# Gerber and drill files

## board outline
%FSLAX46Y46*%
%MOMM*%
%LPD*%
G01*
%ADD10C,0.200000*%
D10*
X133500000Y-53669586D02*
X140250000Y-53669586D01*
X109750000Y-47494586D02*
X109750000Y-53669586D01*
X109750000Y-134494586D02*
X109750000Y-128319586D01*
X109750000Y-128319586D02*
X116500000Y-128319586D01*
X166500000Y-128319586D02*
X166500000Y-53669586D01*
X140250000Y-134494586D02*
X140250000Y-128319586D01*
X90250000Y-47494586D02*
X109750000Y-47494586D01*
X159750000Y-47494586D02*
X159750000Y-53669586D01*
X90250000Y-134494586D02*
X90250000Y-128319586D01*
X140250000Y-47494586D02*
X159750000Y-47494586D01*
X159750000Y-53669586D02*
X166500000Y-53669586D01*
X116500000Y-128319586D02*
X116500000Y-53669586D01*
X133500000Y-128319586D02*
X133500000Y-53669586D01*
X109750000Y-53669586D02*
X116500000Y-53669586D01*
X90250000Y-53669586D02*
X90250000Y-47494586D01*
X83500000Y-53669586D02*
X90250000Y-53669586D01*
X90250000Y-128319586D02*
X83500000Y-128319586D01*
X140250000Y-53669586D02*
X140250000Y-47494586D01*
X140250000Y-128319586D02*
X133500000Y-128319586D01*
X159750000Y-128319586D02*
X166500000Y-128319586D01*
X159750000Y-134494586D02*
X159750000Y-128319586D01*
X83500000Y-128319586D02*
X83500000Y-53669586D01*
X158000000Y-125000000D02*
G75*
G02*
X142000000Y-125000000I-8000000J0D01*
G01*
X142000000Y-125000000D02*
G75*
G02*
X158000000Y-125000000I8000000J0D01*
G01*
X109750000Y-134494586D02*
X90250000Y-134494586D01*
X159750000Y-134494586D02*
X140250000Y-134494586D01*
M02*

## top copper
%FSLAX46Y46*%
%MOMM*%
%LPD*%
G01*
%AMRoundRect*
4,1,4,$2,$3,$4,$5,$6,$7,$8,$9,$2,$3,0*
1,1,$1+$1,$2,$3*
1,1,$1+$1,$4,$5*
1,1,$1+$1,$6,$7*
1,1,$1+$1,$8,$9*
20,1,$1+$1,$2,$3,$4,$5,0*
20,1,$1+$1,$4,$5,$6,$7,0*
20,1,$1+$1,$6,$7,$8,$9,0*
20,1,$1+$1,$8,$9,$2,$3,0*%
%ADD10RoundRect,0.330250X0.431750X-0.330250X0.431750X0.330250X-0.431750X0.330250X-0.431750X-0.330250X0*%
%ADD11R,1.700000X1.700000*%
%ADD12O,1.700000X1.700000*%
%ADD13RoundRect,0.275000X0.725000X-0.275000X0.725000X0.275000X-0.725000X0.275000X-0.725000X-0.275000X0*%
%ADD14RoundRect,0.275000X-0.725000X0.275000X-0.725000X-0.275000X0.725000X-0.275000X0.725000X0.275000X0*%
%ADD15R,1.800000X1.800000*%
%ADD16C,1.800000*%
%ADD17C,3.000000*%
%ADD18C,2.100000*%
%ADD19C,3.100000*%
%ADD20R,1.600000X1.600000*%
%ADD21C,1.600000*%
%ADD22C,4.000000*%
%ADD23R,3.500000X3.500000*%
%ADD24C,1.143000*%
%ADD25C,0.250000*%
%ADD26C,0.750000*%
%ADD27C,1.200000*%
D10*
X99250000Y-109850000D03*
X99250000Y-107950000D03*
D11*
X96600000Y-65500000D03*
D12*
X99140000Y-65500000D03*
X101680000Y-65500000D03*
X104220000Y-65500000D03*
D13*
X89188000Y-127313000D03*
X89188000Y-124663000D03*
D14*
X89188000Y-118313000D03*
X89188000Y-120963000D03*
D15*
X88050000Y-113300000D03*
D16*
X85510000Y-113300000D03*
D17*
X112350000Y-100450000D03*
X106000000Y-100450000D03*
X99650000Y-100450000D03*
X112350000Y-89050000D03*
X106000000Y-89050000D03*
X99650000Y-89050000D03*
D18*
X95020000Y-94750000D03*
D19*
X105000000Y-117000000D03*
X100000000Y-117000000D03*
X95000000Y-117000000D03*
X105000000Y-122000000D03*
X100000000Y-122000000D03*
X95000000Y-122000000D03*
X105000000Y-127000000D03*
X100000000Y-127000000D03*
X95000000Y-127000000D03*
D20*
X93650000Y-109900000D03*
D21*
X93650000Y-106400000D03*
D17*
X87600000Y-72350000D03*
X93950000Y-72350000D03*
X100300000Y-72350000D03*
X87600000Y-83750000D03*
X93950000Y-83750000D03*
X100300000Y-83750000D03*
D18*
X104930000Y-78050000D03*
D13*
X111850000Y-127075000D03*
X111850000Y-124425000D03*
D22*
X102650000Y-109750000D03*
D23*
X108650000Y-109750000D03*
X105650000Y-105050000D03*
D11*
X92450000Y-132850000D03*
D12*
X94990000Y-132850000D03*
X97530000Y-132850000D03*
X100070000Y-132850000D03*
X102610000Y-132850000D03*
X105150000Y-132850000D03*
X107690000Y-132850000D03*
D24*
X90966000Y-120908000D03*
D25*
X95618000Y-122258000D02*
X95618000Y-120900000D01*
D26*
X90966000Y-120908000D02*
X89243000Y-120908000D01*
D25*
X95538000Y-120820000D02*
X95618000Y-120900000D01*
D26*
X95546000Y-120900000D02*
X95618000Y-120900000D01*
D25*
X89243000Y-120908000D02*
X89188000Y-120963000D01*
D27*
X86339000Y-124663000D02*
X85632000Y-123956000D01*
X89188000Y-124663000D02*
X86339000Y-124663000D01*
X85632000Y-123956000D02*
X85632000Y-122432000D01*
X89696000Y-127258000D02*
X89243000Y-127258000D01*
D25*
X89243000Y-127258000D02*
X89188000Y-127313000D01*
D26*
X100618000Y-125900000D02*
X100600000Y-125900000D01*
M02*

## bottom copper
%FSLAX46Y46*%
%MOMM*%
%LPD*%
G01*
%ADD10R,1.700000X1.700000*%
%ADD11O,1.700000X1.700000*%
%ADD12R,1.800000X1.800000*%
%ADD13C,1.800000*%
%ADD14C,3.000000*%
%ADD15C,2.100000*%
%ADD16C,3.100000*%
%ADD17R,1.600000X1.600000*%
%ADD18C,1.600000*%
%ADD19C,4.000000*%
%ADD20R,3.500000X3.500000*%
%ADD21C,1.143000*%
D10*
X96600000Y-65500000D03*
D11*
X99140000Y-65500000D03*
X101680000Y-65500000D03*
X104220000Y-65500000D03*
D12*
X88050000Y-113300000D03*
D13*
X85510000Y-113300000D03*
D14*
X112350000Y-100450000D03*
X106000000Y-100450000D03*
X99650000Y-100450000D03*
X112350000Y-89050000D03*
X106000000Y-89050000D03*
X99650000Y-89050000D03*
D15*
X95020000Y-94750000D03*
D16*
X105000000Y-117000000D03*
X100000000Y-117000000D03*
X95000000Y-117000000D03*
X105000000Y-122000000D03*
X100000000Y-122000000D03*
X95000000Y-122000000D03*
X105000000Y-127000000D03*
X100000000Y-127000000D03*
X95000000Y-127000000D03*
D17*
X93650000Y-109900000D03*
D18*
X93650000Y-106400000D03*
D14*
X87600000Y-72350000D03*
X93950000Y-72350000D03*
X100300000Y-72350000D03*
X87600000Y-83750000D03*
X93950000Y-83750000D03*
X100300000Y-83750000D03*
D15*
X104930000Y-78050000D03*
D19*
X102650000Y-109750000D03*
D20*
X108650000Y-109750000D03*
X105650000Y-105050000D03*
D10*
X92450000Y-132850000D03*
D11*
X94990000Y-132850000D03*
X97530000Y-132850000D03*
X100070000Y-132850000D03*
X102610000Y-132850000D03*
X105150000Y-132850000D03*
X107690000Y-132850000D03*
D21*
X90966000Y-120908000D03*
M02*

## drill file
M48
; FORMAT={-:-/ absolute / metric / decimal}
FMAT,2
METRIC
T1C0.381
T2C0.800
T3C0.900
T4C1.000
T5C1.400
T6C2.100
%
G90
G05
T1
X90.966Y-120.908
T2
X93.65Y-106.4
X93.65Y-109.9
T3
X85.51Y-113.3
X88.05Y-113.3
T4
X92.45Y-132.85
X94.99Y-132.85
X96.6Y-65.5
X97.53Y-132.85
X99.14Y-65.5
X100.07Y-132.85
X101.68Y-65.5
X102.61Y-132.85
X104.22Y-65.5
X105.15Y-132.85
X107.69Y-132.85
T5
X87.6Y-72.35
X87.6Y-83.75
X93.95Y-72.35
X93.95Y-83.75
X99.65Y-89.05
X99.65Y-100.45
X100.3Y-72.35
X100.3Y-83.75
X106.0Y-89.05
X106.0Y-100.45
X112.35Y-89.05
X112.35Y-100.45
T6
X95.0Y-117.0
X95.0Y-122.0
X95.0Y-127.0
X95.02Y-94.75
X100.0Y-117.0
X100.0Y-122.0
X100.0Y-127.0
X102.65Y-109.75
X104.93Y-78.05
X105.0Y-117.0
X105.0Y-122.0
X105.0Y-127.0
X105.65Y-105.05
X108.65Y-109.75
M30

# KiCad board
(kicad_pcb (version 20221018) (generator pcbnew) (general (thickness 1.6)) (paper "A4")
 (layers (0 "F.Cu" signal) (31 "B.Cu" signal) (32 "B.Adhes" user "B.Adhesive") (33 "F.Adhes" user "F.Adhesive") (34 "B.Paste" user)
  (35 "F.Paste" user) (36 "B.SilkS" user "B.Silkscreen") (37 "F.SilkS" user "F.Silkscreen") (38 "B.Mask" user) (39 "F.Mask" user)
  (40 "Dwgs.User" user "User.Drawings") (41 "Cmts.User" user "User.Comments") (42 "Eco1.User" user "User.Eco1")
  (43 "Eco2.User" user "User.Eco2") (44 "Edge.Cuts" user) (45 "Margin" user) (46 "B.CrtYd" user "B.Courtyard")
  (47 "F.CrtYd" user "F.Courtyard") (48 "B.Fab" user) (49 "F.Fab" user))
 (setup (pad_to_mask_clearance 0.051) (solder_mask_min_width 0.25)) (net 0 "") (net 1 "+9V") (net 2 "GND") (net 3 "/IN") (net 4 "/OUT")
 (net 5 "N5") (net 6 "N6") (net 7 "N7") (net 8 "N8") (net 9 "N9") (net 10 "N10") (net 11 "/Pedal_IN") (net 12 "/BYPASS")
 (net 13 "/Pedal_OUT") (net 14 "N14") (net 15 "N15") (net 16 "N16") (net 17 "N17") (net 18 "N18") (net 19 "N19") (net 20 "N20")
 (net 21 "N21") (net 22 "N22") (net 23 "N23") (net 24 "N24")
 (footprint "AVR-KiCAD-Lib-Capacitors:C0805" (layer "F.Cu") (at 99.25 108.9 90)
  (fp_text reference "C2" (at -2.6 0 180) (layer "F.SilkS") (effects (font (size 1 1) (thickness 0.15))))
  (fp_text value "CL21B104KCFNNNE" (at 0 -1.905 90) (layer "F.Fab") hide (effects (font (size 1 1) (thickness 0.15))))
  (pad "1" smd roundrect (at -0.95 0 90) (size 1.321 1.524) (layers "F.Cu" "F.Paste" "F.Mask") (roundrect_rratio 0.25) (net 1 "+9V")
   (solder_mask_margin 0.102))
  (pad "2" smd roundrect (at 0.95 0 90) (size 1.321 1.524) (layers "F.Cu" "F.Paste" "F.Mask") (roundrect_rratio 0.25) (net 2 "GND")
   (solder_mask_margin 0.102)))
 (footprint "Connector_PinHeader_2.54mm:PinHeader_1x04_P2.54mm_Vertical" (layer "F.Cu") (at 96.6 65.5 90)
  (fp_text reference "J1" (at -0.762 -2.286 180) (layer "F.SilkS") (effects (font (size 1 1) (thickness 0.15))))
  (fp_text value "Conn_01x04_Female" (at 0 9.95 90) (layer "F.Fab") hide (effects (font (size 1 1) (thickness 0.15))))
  (pad "1" thru_hole rect (at 0 0 90) (size 1.7 1.7) (drill 1) (layers "*.Cu" "*.Mask") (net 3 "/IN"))
  (pad "2" thru_hole oval (at 0 2.54 90) (size 1.7 1.7) (drill 1) (layers "*.Cu" "*.Mask") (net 2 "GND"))
  (pad "3" thru_hole oval (at 0 5.08 90) (size 1.7 1.7) (drill 1) (layers "*.Cu" "*.Mask") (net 1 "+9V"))
  (pad "4" thru_hole oval (at 0 7.62 90) (size 1.7 1.7) (drill 1) (layers "*.Cu" "*.Mask") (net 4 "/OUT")))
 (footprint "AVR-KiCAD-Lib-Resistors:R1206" (layer "F.Cu") (at 89.188 125.988 90)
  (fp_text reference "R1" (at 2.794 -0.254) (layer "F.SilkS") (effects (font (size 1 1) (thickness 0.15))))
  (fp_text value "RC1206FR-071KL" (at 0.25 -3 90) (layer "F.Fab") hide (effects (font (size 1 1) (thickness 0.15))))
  (pad "1" smd roundrect (at -1.325 0 90) (size 1.1 2) (layers "F.Cu" "F.Paste" "F.Mask") (roundrect_rratio 0.25) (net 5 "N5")
   (solder_mask_margin 0.102))
  (pad "2" smd roundrect (at 1.325 0 90) (size 1.1 2) (layers "F.Cu" "F.Paste" "F.Mask") (roundrect_rratio 0.25) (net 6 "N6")
   (solder_mask_margin 0.102)))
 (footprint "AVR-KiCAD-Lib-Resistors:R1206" (layer "F.Cu") (at 89.188 119.638 -90)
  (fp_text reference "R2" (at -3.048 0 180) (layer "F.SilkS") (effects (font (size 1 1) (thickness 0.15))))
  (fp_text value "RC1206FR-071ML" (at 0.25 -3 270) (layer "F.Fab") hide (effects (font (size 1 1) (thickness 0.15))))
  (pad "1" smd roundrect (at -1.325 0 270) (size 1.1 2) (layers "F.Cu" "F.Paste" "F.Mask") (roundrect_rratio 0.25) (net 3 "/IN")
   (solder_mask_margin 0.102))
  (pad "2" smd roundrect (at 1.325 0 270) (size 1.1 2) (layers "F.Cu" "F.Paste" "F.Mask") (roundrect_rratio 0.25) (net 2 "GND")
   (solder_mask_margin 0.102)))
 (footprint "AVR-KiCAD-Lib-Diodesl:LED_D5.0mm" (layer "F.Cu") (at 88.05 113.3 180)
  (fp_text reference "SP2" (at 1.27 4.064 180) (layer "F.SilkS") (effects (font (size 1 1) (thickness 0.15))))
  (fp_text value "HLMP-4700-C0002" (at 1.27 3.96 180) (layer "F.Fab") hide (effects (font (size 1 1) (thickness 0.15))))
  (pad "1" thru_hole rect (at 0 0 180) (size 1.8 1.8) (drill 0.9) (layers "*.Cu" "*.Mask") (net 6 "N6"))
  (pad "2" thru_hole circle (at 2.54 0 180) (size 1.8 1.8) (drill 0.9) (layers "*.Cu" "*.Mask") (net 1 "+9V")))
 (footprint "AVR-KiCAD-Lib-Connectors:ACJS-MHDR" (layer "F.Cu") (at 106 94.75)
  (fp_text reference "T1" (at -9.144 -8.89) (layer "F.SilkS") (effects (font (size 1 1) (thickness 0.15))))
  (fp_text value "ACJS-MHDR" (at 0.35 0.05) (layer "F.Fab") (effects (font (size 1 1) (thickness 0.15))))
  (pad "1" thru_hole circle (at 6.35 5.7) (size 3 3) (drill 1.4) (layers "*.Cu" "*.Mask") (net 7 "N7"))
  (pad "2" thru_hole circle (at 0 5.7) (size 3 3) (drill 1.4) (layers "*.Cu" "*.Mask") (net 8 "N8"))
  (pad "3" thru_hole circle (at -6.35 5.7) (size 3 3) (drill 1.4) (layers "*.Cu" "*.Mask") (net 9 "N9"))
  (pad "4" thru_hole circle (at 6.35 -5.7) (size 3 3) (drill 1.4) (layers "*.Cu" "*.Mask") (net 2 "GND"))
  (pad "5" thru_hole circle (at 0 -5.7) (size 3 3) (drill 1.4) (layers "*.Cu" "*.Mask") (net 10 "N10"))
  (pad "6" thru_hole circle (at -6.35 -5.7) (size 3 3) (drill 1.4) (layers "*.Cu" "*.Mask") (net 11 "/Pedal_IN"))
  (pad "7" thru_hole circle (at -10.98 0) (size 2.1 2.1) (drill 2.1) (layers "*.Cu" "*.Mask")))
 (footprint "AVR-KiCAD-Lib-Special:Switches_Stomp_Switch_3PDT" (layer "F.Cu") (at 100 122)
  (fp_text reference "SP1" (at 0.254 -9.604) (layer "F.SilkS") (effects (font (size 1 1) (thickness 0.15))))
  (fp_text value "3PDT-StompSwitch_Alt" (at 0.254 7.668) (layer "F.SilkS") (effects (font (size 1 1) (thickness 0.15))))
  (pad "1" thru_hole circle (at 5 -5) (size 3.1 3.1) (drill 2.1) (layers "*.Cu" "*.Mask" "F.SilkS") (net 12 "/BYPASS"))
  (pad "2" thru_hole circle (at 0 -5) (size 3.1 3.1) (drill 2.1) (layers "*.Cu" "*.Mask" "F.SilkS") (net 12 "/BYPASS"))
  (pad "3" thru_hole circle (at -5 -5) (size 3.1 3.1) (drill 2.1) (layers "*.Cu" "*.Mask" "F.SilkS") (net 3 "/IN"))
  (pad "4" thru_hole circle (at 5 0) (size 3.1 3.1) (drill 2.1) (layers "*.Cu" "*.Mask" "F.SilkS") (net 11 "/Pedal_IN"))
  (pad "5" thru_hole circle (at 0 0) (size 3.1 3.1) (drill 2.1) (layers "*.Cu" "*.Mask" "F.SilkS") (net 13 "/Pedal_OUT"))
  (pad "6" thru_hole circle (at -5 0) (size 3.1 3.1) (drill 2.1) (layers "*.Cu" "*.Mask" "F.SilkS") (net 2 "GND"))
  (pad "7" thru_hole circle (at 5 5) (size 3.1 3.1) (drill 2.1) (layers "*.Cu" "*.Mask" "F.SilkS") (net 3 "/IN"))
  (pad "8" thru_hole circle (at 0 5) (size 3.1 3.1) (drill 2.1) (layers "*.Cu" "*.Mask" "F.SilkS") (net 4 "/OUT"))
  (pad "9" thru_hole circle (at -5 5) (size 3.1 3.1) (drill 2.1) (layers "*.Cu" "*.Mask" "F.SilkS") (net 5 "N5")))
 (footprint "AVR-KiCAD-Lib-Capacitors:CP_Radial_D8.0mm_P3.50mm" (layer "F.Cu") (at 93.65 109.9 90)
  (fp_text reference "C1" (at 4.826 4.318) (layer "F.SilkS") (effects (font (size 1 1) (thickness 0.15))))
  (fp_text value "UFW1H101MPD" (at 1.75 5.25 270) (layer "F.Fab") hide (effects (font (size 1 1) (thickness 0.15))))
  (pad "1" thru_hole rect (at 0 0 90) (size 1.6 1.6) (drill 0.8) (layers "*.Cu" "*.Mask") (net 1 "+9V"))
  (pad "2" thru_hole circle (at 3.5 0 90) (size 1.6 1.6) (drill 0.8) (layers "*.Cu" "*.Mask") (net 2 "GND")))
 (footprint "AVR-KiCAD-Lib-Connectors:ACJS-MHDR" (layer "F.Cu") (at 93.95 78.05 180)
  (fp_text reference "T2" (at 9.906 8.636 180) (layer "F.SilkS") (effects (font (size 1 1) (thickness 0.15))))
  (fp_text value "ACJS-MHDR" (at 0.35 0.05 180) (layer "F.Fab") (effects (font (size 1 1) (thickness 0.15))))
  (pad "1" thru_hole circle (at 6.35 5.7 180) (size 3 3) (drill 1.4) (layers "*.Cu" "*.Mask") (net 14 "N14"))
  (pad "2" thru_hole circle (at 0 5.7 180) (size 3 3) (drill 1.4) (layers "*.Cu" "*.Mask") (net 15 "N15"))
  (pad "3" thru_hole circle (at -6.35 5.7 180) (size 3 3) (drill 1.4) (layers "*.Cu" "*.Mask") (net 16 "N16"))
  (pad "4" thru_hole circle (at 6.35 -5.7 180) (size 3 3) (drill 1.4) (layers "*.Cu" "*.Mask") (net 2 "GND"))
  (pad "5" thru_hole circle (at 0 -5.7 180) (size 3 3) (drill 1.4) (layers "*.Cu" "*.Mask") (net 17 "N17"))
  (pad "6" thru_hole circle (at -6.35 -5.7 180) (size 3 3) (drill 1.4) (layers "*.Cu" "*.Mask") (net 13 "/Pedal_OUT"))
  (pad "7" thru_hole circle (at -10.98 0 180) (size 2.1 2.1) (drill 2.1) (layers "*.Cu" "*.Mask")))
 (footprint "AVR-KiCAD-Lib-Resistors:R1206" (layer "F.Cu") (at 111.85 125.75 90)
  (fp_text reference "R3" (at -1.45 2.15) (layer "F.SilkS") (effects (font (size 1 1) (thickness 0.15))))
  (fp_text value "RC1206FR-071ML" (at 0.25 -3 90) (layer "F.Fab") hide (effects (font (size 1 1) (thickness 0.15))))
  (pad "1" smd roundrect (at -1.325 0 90) (size 1.1 2) (layers "F.Cu" "F.Paste" "F.Mask") (roundrect_rratio 0.25) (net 4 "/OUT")
   (solder_mask_margin 0.102))
  (pad "2" smd roundrect (at 1.325 0 90) (size 1.1 2) (layers "F.Cu" "F.Paste" "F.Mask") (roundrect_rratio 0.25) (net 2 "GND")
   (solder_mask_margin 0.102)))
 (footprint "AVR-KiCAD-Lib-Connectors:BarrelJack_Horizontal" (layer "F.Cu") (at 102.65 109.75 180)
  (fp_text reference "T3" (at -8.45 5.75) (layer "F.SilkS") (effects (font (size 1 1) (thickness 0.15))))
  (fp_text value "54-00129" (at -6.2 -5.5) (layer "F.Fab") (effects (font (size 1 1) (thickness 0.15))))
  (pad "1" thru_hole circle (at 0 0 180) (size 4 4) (drill 2.1) (layers "*.Cu" "*.Mask") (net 1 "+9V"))
  (pad "2" thru_hole rect (at -6 0 180) (size 3.5 3.5) (drill 2.1) (layers "*.Cu" "*.Mask") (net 2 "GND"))
  (pad "3" thru_hole rect (at -3 4.7 180) (size 3.5 3.5) (drill 2.1) (layers "*.Cu" "*.Mask") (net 2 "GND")))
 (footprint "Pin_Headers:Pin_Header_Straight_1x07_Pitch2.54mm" (layer "F.Cu") (at 92.45 132.85 90)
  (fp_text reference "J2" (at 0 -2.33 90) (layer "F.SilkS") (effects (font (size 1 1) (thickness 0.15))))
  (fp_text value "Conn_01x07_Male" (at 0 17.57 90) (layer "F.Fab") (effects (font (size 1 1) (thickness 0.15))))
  (pad "1" thru_hole rect (at 0 0 90) (size 1.7 1.7) (drill 1) (layers "*.Cu" "*.Mask") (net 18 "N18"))
  (pad "2" thru_hole oval (at 0 2.54 90) (size 1.7 1.7) (drill 1) (layers "*.Cu" "*.Mask") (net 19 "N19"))
  (pad "3" thru_hole oval (at 0 5.08 90) (size 1.7 1.7) (drill 1) (layers "*.Cu" "*.Mask") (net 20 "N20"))
  (pad "4" thru_hole oval (at 0 7.62 90) (size 1.7 1.7) (drill 1) (layers "*.Cu" "*.Mask") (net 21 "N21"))
  (pad "5" thru_hole oval (at 0 10.16 90) (size 1.7 1.7) (drill 1) (layers "*.Cu" "*.Mask") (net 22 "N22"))
  (pad "6" thru_hole oval (at 0 12.7 90) (size 1.7 1.7) (drill 1) (layers "*.Cu" "*.Mask") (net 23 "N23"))
  (pad "7" thru_hole oval (at 0 15.24 90) (size 1.7 1.7) (drill 1) (layers "*.Cu" "*.Mask") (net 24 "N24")))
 (gr_line (start 133.5 53.669586) (end 140.25 53.669586) (stroke (width 0.2) (type solid)) (layer "Edge.Cuts"))
 (gr_line (start 109.75 47.494586) (end 109.75 53.669586) (stroke (width 0.2) (type solid)) (layer "Edge.Cuts"))
 (gr_line (start 109.75 134.494586) (end 109.75 128.319586) (stroke (width 0.2) (type solid)) (layer "Edge.Cuts"))
 (gr_line (start 109.75 128.319586) (end 116.5 128.319586) (stroke (width 0.2) (type solid)) (layer "Edge.Cuts"))
 (gr_line (start 166.5 128.319586) (end 166.5 53.669586) (stroke (width 0.2) (type solid)) (layer "Edge.Cuts"))
 (gr_line (start 140.25 134.494586) (end 140.25 128.319586) (stroke (width 0.2) (type solid)) (layer "Edge.Cuts"))
 (gr_line (start 90.25 47.494586) (end 109.75 47.494586) (stroke (width 0.2) (type solid)) (layer "Edge.Cuts"))
 (gr_line (start 159.75 47.494586) (end 159.75 53.669586) (stroke (width 0.2) (type solid)) (layer "Edge.Cuts"))
 (gr_line (start 90.25 134.494586) (end 90.25 128.319586) (stroke (width 0.2) (type solid)) (layer "Edge.Cuts"))
 (gr_line (start 140.25 47.494586) (end 159.75 47.494586) (stroke (width 0.2) (type solid)) (layer "Edge.Cuts"))
 (gr_line (start 159.75 53.669586) (end 166.5 53.669586) (stroke (width 0.2) (type solid)) (layer "Edge.Cuts"))
 (gr_line (start 116.5 128.319586) (end 116.5 53.669586) (stroke (width 0.2) (type solid)) (layer "Edge.Cuts"))
 (gr_line (start 133.5 128.319586) (end 133.5 53.669586) (stroke (width 0.2) (type solid)) (layer "Edge.Cuts"))
 (gr_line (start 109.75 53.669586) (end 116.5 53.669586) (stroke (width 0.2) (type solid)) (layer "Edge.Cuts"))
 (gr_line (start 90.25 53.669586) (end 90.25 47.494586) (stroke (width 0.2) (type solid)) (layer "Edge.Cuts"))
 (gr_line (start 83.5 53.669586) (end 90.25 53.669586) (stroke (width 0.2) (type solid)) (layer "Edge.Cuts"))
 (gr_line (start 90.25 128.319586) (end 83.5 128.319586) (stroke (width 0.2) (type solid)) (layer "Edge.Cuts"))
 (gr_line (start 140.25 53.669586) (end 140.25 47.494586) (stroke (width 0.2) (type solid)) (layer "Edge.Cuts"))
 (gr_line (start 140.25 128.319586) (end 133.5 128.319586) (stroke (width 0.2) (type solid)) (layer "Edge.Cuts"))
 (gr_line (start 159.75 128.319586) (end 166.5 128.319586) (stroke (width 0.2) (type solid)) (layer "Edge.Cuts"))
 (gr_line (start 159.75 134.494586) (end 159.75 128.319586) (stroke (width 0.2) (type solid)) (layer "Edge.Cuts"))
 (gr_line (start 83.5 128.319586) (end 83.5 53.669586) (stroke (width 0.2) (type solid)) (layer "Edge.Cuts"))
 (gr_circle (center 150 125) (end 158 125) (stroke (width 0.2) (type solid)) (fill none) (layer "Edge.Cuts"))
 (gr_line (start 109.75 134.494586) (end 90.25 134.494586) (stroke (width 0.2) (type solid)) (layer "Edge.Cuts"))
 (gr_line (start 159.75 134.494586) (end 140.25 134.494586) (stroke (width 0.2) (type solid)) (layer "Edge.Cuts"))
 (segment (start 95.618 122.258) (end 95.618 120.9) (width 0.25) (layer "F.Cu") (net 2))
 (segment (start 90.966 120.908) (end 89.243 120.908) (width 0.75) (layer "F.Cu") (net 2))
 (segment (start 95.538 120.82) (end 95.618 120.9) (width 0.25) (layer "F.Cu") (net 2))
 (segment (start 95.546 120.9) (end 95.618 120.9) (width 0.75) (layer "F.Cu") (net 2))
 (segment (start 89.243 120.908) (end 89.188 120.963) (width 0.25) (layer "F.Cu") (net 2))
 (via (at 90.966 120.908) (size 1.143) (drill 0.381) (layers "F.Cu" "B.Cu") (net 2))
 (segment (start 86.339 124.663) (end 85.632 123.956) (width 1.2) (layer "F.Cu") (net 6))
 (segment (start 89.188 124.663) (end 86.339 124.663) (width 1.2) (layer "F.Cu") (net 6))
 (segment (start 85.632 123.956) (end 85.632 122.432) (width 1.2) (layer "F.Cu") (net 6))
 (segment (start 89.696 127.258) (end 89.243 127.258) (width 1.2) (layer "F.Cu") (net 5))
 (segment (start 89.243 127.258) (end 89.188 127.313) (width 0.25) (layer "F.Cu") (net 5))
 (segment (start 100.618 125.9) (end 100.6 125.9) (width 0.75) (layer "F.Cu") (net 4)))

